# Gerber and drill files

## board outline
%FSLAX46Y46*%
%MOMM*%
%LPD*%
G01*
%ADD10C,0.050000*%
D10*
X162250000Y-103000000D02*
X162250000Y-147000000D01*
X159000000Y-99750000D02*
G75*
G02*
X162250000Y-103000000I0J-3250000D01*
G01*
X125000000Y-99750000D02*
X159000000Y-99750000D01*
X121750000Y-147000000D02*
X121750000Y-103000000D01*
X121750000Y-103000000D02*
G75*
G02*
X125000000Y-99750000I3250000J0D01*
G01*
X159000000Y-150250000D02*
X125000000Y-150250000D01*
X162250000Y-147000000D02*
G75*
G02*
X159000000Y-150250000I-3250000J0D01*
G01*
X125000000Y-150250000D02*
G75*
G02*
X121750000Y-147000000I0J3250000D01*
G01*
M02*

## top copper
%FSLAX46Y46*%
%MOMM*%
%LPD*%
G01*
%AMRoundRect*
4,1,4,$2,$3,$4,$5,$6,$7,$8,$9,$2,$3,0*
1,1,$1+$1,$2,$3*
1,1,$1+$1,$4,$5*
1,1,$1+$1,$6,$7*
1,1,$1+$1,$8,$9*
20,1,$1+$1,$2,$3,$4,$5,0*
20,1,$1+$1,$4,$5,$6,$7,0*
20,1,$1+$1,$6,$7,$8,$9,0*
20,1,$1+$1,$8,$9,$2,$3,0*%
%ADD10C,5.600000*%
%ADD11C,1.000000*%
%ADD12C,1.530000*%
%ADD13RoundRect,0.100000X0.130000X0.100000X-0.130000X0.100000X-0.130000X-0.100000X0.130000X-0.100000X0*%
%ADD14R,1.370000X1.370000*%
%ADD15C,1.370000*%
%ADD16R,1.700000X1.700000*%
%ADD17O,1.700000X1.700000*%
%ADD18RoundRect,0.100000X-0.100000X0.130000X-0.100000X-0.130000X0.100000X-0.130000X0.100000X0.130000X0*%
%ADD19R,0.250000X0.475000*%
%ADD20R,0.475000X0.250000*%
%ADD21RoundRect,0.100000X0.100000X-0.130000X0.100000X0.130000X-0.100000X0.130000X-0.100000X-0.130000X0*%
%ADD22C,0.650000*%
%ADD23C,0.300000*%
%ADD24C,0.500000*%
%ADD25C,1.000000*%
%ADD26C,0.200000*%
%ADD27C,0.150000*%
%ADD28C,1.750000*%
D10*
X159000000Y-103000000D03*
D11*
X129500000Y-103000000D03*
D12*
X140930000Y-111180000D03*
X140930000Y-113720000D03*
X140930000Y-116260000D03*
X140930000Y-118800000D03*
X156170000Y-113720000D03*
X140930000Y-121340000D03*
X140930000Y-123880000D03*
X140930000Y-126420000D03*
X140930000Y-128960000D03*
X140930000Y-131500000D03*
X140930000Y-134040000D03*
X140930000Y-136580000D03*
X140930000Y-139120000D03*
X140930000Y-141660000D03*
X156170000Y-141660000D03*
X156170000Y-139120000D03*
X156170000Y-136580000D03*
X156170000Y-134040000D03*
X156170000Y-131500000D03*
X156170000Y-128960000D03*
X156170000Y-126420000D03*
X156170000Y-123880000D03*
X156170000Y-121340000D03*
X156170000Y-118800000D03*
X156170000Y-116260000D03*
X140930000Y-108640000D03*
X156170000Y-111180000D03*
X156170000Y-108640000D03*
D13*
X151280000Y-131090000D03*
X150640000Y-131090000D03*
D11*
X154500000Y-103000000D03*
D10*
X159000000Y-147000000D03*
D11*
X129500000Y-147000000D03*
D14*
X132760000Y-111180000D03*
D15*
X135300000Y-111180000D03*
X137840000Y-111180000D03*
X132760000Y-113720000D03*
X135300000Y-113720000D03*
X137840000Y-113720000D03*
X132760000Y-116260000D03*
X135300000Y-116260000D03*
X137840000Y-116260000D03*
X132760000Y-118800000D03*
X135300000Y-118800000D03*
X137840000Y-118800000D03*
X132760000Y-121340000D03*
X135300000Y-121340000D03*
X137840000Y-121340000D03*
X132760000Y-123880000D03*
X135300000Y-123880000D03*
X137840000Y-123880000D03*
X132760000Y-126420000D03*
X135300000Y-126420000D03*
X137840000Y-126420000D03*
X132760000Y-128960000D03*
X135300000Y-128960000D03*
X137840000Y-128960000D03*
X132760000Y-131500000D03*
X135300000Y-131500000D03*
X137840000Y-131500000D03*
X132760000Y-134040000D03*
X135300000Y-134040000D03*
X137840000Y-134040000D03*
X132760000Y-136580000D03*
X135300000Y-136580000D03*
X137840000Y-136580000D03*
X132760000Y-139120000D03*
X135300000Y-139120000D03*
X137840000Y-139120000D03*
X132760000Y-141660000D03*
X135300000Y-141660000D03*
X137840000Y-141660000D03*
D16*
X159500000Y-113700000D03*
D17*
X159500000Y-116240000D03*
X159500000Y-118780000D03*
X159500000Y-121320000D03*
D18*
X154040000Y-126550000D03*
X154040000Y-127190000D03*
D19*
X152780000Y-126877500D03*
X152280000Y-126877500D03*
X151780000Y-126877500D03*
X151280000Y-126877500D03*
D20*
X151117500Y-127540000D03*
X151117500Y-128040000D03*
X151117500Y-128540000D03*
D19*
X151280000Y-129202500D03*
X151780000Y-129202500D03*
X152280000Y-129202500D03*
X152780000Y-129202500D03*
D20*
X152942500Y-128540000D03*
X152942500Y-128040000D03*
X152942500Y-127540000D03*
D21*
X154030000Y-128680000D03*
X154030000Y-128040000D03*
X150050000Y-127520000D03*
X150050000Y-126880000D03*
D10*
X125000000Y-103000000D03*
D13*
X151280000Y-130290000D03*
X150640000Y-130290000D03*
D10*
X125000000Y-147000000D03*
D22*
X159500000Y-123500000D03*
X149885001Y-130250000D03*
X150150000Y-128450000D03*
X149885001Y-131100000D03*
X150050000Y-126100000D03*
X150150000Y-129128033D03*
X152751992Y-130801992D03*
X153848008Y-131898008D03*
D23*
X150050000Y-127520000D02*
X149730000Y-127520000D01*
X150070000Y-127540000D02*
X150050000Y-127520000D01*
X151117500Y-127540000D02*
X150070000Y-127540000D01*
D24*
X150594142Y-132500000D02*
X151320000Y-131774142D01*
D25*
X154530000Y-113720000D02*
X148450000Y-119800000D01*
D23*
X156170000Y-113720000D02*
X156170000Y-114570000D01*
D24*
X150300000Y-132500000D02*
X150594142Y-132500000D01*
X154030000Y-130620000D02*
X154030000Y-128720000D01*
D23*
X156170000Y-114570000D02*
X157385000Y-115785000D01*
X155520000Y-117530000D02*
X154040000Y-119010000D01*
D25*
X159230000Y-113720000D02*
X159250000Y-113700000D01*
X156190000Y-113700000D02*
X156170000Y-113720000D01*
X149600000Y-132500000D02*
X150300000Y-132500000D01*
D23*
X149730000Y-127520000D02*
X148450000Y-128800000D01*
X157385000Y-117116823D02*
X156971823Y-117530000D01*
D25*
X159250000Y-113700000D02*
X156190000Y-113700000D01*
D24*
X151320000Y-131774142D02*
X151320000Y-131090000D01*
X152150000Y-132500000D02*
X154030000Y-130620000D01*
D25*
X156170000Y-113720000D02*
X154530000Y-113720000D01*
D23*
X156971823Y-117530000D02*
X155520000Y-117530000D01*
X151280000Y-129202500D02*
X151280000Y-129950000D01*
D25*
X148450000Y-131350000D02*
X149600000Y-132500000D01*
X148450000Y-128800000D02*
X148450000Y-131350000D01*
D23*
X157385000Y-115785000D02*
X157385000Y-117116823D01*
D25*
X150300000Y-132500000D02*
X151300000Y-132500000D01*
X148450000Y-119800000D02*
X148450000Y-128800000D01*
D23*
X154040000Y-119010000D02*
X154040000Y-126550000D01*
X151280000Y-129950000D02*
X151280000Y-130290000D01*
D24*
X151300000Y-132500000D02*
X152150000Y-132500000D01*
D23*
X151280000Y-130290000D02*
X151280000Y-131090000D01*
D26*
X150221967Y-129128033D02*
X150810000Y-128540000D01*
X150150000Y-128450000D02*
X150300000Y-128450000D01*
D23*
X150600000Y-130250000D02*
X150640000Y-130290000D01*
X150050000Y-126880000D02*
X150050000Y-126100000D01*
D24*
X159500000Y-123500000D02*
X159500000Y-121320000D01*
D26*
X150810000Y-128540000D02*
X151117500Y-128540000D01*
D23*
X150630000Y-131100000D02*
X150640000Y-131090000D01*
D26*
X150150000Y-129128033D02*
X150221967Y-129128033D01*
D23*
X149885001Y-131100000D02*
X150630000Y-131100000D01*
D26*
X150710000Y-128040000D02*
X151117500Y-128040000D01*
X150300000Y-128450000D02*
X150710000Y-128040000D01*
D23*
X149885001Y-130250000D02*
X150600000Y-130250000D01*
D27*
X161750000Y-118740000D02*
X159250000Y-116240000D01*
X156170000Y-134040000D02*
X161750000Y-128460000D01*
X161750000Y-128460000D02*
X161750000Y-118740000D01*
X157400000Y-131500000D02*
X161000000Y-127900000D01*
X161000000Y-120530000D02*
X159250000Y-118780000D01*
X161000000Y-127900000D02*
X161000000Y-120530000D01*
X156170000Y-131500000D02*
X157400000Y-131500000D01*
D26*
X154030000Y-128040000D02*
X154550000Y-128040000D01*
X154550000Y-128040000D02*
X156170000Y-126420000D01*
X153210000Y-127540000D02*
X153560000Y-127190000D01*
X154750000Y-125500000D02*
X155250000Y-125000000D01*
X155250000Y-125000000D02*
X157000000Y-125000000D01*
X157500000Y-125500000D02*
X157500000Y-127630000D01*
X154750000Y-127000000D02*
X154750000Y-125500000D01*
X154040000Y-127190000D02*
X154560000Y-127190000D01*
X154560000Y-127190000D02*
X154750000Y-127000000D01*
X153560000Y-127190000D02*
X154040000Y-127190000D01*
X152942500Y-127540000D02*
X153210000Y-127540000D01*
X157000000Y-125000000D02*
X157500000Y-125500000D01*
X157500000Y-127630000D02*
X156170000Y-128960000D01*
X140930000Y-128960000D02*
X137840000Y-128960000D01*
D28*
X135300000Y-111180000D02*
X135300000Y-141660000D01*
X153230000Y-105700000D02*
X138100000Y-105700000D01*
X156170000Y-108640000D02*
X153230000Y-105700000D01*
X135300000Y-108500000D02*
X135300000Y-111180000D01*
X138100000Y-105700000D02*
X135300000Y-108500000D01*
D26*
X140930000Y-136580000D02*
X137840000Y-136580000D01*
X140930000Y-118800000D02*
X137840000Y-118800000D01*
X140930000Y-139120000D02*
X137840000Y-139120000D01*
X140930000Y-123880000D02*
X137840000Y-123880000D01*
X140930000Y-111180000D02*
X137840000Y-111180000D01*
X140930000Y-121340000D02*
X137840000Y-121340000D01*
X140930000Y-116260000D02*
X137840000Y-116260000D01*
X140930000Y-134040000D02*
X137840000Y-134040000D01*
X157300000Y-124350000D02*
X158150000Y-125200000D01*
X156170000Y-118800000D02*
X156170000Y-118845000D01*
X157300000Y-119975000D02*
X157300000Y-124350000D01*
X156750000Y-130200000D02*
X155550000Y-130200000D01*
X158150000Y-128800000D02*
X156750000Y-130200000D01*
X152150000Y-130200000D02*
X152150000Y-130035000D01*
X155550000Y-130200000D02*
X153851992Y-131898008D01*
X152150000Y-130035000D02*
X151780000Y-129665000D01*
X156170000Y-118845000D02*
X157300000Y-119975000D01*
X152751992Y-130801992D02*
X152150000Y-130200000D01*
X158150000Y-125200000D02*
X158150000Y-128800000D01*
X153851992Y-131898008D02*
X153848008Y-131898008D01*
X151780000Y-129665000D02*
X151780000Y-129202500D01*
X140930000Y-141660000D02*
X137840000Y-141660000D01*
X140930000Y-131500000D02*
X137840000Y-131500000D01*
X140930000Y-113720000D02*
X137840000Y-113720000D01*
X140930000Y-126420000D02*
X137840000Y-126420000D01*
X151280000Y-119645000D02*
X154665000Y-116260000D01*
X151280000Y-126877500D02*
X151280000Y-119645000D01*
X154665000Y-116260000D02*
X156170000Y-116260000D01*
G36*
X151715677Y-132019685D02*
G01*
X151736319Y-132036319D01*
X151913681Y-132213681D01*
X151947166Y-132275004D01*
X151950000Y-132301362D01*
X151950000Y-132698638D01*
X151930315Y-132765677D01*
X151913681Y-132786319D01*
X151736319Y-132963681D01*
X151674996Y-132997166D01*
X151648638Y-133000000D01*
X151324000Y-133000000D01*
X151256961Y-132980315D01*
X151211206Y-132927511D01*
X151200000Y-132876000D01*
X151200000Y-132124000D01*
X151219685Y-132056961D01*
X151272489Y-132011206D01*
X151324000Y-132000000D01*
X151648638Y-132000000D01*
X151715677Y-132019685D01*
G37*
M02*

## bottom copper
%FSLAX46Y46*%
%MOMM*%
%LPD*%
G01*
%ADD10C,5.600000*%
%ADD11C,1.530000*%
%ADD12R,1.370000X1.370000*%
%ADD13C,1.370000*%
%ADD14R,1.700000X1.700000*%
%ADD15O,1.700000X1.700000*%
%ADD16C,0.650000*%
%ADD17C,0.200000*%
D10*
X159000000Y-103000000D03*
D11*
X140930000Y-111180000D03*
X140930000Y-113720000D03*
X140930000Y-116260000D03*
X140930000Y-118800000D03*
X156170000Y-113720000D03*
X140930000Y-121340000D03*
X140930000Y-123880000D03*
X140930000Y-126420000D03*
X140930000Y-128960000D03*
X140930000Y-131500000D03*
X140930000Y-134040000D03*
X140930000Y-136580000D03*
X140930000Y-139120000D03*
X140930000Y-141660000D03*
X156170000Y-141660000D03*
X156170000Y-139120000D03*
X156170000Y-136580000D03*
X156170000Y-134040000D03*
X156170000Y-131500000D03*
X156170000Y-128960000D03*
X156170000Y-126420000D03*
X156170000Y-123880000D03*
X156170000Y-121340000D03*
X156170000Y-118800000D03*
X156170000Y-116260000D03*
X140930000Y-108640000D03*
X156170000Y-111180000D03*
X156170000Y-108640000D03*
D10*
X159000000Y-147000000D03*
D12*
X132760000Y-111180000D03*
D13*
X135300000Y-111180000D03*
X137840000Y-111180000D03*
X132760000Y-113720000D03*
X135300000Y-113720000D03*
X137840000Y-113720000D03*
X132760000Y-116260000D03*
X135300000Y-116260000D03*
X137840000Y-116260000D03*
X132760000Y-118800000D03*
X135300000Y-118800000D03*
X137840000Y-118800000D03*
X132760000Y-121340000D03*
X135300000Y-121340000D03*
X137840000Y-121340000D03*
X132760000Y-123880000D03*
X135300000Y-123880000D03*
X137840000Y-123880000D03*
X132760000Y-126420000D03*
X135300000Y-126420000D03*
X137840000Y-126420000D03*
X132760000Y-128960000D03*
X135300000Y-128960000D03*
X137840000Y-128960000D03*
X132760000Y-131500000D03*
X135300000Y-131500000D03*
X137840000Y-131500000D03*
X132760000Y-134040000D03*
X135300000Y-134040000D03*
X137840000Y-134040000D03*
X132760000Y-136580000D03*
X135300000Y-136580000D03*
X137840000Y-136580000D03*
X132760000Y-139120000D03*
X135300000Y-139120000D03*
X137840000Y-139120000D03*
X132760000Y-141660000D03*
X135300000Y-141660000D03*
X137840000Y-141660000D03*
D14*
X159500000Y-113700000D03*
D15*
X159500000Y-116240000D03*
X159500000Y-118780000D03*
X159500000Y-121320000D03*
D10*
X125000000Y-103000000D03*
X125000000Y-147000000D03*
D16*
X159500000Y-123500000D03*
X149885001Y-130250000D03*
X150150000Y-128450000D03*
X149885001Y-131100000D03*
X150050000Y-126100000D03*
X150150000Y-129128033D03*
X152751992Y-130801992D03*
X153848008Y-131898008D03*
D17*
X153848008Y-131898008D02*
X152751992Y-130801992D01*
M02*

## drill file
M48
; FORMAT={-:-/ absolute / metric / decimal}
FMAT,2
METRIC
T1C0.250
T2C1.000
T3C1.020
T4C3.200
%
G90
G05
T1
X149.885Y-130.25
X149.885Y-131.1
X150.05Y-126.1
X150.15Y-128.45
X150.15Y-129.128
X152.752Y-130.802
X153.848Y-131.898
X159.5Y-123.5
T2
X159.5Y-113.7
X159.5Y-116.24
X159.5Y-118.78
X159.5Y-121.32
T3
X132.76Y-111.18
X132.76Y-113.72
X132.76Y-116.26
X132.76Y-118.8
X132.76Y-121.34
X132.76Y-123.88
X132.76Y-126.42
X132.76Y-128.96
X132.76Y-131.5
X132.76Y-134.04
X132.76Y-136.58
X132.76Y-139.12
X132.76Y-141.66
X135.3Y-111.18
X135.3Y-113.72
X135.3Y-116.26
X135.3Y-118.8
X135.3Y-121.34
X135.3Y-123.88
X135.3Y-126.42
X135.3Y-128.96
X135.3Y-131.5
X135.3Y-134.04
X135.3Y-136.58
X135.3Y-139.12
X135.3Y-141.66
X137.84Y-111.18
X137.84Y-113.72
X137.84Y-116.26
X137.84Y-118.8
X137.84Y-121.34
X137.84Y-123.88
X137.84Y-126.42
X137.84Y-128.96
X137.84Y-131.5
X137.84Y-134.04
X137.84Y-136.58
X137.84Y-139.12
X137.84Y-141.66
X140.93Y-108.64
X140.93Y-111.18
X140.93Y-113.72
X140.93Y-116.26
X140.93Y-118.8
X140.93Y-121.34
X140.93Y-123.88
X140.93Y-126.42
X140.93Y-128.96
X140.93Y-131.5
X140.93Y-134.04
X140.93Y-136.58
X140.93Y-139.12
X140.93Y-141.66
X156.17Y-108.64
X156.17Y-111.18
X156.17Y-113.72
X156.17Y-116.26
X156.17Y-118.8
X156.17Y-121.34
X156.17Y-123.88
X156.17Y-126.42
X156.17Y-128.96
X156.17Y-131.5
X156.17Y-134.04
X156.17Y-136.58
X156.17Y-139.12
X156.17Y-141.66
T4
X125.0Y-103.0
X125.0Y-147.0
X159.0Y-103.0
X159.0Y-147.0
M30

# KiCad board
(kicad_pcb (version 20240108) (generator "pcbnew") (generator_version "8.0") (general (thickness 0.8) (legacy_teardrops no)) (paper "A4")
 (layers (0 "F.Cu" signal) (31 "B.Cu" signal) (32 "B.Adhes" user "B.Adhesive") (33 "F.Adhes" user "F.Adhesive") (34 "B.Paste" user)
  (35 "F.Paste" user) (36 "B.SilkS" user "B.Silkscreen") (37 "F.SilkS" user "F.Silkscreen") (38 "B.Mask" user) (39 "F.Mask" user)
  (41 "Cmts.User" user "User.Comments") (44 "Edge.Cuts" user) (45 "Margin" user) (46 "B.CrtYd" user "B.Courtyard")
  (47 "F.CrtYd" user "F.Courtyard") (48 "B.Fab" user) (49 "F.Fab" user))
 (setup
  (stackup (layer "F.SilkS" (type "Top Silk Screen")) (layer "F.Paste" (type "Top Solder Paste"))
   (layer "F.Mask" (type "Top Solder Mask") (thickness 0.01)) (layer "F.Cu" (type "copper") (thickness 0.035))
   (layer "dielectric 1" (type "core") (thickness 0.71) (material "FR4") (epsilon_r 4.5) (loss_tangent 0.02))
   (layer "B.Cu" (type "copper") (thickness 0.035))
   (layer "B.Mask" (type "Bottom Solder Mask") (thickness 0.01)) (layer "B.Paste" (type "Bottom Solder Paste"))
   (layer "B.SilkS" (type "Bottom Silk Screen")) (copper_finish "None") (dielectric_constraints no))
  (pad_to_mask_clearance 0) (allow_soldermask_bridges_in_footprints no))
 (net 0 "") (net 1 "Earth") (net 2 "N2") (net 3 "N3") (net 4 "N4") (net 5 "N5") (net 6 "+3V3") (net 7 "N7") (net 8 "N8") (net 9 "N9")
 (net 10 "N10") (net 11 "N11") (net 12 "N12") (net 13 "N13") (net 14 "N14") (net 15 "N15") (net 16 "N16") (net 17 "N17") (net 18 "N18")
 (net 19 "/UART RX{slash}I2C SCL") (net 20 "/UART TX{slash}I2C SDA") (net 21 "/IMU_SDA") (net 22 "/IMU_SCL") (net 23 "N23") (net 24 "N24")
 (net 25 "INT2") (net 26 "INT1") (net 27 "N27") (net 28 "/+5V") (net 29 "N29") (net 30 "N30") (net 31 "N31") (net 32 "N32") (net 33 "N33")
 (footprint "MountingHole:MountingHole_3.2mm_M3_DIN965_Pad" (layer "F.Cu") (at 159 103)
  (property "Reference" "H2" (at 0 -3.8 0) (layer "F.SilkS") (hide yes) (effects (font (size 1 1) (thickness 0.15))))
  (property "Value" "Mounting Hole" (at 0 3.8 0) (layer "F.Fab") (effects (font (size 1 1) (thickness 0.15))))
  (pad "1" thru_hole circle (at 0 0) (size 5.6 5.6) (drill 3.2) (layers "*.Cu" "*.Mask") (remove_unused_layers no) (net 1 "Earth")))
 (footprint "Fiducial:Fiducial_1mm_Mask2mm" (layer "F.Cu") (at 129.5 103)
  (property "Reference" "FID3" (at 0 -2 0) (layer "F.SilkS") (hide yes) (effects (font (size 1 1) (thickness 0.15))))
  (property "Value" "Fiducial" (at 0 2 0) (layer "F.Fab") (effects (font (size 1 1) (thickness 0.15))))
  (pad "" smd circle (at 0 0) (size 1 1) (layers "F.Cu" "F.Mask") (solder_mask_margin 0.5) (clearance 0.5)))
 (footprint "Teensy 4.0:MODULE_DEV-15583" (layer "F.Cu") (at 148.55 125.15)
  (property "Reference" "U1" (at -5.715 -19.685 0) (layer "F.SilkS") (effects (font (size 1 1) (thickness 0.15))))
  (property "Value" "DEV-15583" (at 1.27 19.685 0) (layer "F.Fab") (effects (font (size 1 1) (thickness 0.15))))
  (pad "0" thru_hole circle (at -7.62 -13.97) (size 1.53 1.53) (drill 1.02) (layers "*.Cu" "*.Mask") (remove_unused_layers no) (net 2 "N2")
   (solder_mask_margin 0.102))
  (pad "1" thru_hole circle (at -7.62 -11.43) (size 1.53 1.53) (drill 1.02) (layers "*.Cu" "*.Mask") (remove_unused_layers no) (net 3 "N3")
   (solder_mask_margin 0.102))
  (pad "2" thru_hole circle (at -7.62 -8.89) (size 1.53 1.53) (drill 1.02) (layers "*.Cu" "*.Mask") (remove_unused_layers no) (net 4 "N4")
   (solder_mask_margin 0.102))
  (pad "3" thru_hole circle (at -7.62 -6.35) (size 1.53 1.53) (drill 1.02) (layers "*.Cu" "*.Mask") (remove_unused_layers no) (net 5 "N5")
   (solder_mask_margin 0.102))
  (pad "3v3" thru_hole circle (at 7.62 -11.43) (size 1.53 1.53) (drill 1.02) (layers "*.Cu" "*.Mask") (remove_unused_layers no)
   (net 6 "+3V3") (solder_mask_margin 0.102))
  (pad "4" thru_hole circle (at -7.62 -3.81) (size 1.53 1.53) (drill 1.02) (layers "*.Cu" "*.Mask") (remove_unused_layers no) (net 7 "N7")
   (solder_mask_margin 0.102))
  (pad "5" thru_hole circle (at -7.62 -1.27) (size 1.53 1.53) (drill 1.02) (layers "*.Cu" "*.Mask") (remove_unused_layers no) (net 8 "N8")
   (solder_mask_margin 0.102))
  (pad "6" thru_hole circle (at -7.62 1.27) (size 1.53 1.53) (drill 1.02) (layers "*.Cu" "*.Mask") (remove_unused_layers no) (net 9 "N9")
   (solder_mask_margin 0.102))
  (pad "7" thru_hole circle (at -7.62 3.81) (size 1.53 1.53) (drill 1.02) (layers "*.Cu" "*.Mask") (remove_unused_layers no) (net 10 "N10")
   (solder_mask_margin 0.102))
  (pad "8" thru_hole circle (at -7.62 6.35) (size 1.53 1.53) (drill 1.02) (layers "*.Cu" "*.Mask") (remove_unused_layers no) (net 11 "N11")
   (solder_mask_margin 0.102))
  (pad "9" thru_hole circle (at -7.62 8.89) (size 1.53 1.53) (drill 1.02) (layers "*.Cu" "*.Mask") (remove_unused_layers no) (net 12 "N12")
   (solder_mask_margin 0.102))
  (pad "10" thru_hole circle (at -7.62 11.43) (size 1.53 1.53) (drill 1.02) (layers "*.Cu" "*.Mask") (remove_unused_layers no)
   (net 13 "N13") (solder_mask_margin 0.102))
  (pad "11" thru_hole circle (at -7.62 13.97) (size 1.53 1.53) (drill 1.02) (layers "*.Cu" "*.Mask") (remove_unused_layers no)
   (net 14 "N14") (solder_mask_margin 0.102))
  (pad "12" thru_hole circle (at -7.62 16.51) (size 1.53 1.53) (drill 1.02) (layers "*.Cu" "*.Mask") (remove_unused_layers no)
   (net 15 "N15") (solder_mask_margin 0.102))
  (pad "13" thru_hole circle (at 7.62 16.51) (size 1.53 1.53) (drill 1.02) (layers "*.Cu" "*.Mask") (remove_unused_layers no) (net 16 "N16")
   (solder_mask_margin 0.102))
  (pad "14" thru_hole circle (at 7.62 13.97) (size 1.53 1.53) (drill 1.02) (layers "*.Cu" "*.Mask") (remove_unused_layers no) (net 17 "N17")
   (solder_mask_margin 0.102))
  (pad "15" thru_hole circle (at 7.62 11.43) (size 1.53 1.53) (drill 1.02) (layers "*.Cu" "*.Mask") (remove_unused_layers no) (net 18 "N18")
   (solder_mask_margin 0.102))
  (pad "16" thru_hole circle (at 7.62 8.89) (size 1.53 1.53) (drill 1.02) (layers "*.Cu" "*.Mask") (remove_unused_layers no)
   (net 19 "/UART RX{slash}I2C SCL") (solder_mask_margin 0.102))
  (pad "17" thru_hole circle (at 7.62 6.35) (size 1.53 1.53) (drill 1.02) (layers "*.Cu" "*.Mask") (remove_unused_layers no)
   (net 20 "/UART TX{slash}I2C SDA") (solder_mask_margin 0.102))
  (pad "18" thru_hole circle (at 7.62 3.81) (size 1.53 1.53) (drill 1.02) (layers "*.Cu" "*.Mask") (remove_unused_layers no)
   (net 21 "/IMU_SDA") (solder_mask_margin 0.102))
  (pad "19" thru_hole circle (at 7.62 1.27) (size 1.53 1.53) (drill 1.02) (layers "*.Cu" "*.Mask") (remove_unused_layers no)
   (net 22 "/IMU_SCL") (solder_mask_margin 0.102))
  (pad "20" thru_hole circle (at 7.62 -1.27) (size 1.53 1.53) (drill 1.02) (layers "*.Cu" "*.Mask") (remove_unused_layers no) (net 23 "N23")
   (solder_mask_margin 0.102))
  (pad "21" thru_hole circle (at 7.62 -3.81) (size 1.53 1.53) (drill 1.02) (layers "*.Cu" "*.Mask") (remove_unused_layers no) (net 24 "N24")
   (solder_mask_margin 0.102))
  (pad "22" thru_hole circle (at 7.62 -6.35) (size 1.53 1.53) (drill 1.02) (layers "*.Cu" "*.Mask") (remove_unused_layers no)
   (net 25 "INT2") (solder_mask_margin 0.102))
  (pad "23" thru_hole circle (at 7.62 -8.89) (size 1.53 1.53) (drill 1.02) (layers "*.Cu" "*.Mask") (remove_unused_layers no)
   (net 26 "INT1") (solder_mask_margin 0.102))
  (pad "G1" thru_hole circle (at -7.62 -16.51) (size 1.53 1.53) (drill 1.02) (layers "*.Cu" "*.Mask") (remove_unused_layers no)
   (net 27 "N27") (solder_mask_margin 0.102))
  (pad "G3" thru_hole circle (at 7.62 -13.97) (size 1.53 1.53) (drill 1.02) (layers "*.Cu" "*.Mask") (remove_unused_layers no)
   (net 1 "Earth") (solder_mask_margin 0.102))
  (pad "VIN" thru_hole circle (at 7.62 -16.51) (size 1.53 1.53) (drill 1.02) (layers "*.Cu" "*.Mask") (remove_unused_layers no)
   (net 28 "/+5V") (solder_mask_margin 0.102)))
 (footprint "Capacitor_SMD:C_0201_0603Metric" (layer "F.Cu") (at 150.96 131.09 180)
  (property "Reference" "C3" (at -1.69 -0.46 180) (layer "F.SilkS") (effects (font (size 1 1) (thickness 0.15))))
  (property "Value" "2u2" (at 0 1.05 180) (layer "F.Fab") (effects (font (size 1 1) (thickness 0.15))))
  (pad "" smd roundrect (at -0.345 0 180) (size 0.318 0.36) (layers "F.Paste") (roundrect_rratio 0.25))
  (pad "" smd roundrect (at 0.345 0 180) (size 0.318 0.36) (layers "F.Paste") (roundrect_rratio 0.25))
  (pad "1" smd roundrect (at -0.32 0 180) (size 0.46 0.4) (layers "F.Cu" "F.Mask") (roundrect_rratio 0.25) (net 6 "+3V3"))
  (pad "2" smd roundrect (at 0.32 0 180) (size 0.46 0.4) (layers "F.Cu" "F.Mask") (roundrect_rratio 0.25) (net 1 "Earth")))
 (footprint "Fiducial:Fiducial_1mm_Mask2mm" (layer "F.Cu") (at 154.5 103)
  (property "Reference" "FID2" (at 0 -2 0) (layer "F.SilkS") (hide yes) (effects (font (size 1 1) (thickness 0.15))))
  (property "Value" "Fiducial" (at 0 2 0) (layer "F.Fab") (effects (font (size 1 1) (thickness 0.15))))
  (pad "" smd circle (at 0 0) (size 1 1) (layers "F.Cu" "F.Mask") (solder_mask_margin 0.5) (clearance 0.5)))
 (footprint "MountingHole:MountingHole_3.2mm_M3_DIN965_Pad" (layer "F.Cu") (at 159 147)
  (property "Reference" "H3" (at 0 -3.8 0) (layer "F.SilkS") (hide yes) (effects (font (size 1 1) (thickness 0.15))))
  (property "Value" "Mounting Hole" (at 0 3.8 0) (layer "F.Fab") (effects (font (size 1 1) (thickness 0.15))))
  (pad "1" thru_hole circle (at 0 0) (size 5.6 5.6) (drill 3.2) (layers "*.Cu" "*.Mask") (remove_unused_layers no) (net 1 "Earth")))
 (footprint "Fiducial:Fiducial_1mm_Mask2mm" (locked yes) (layer "F.Cu") (at 129.5 147)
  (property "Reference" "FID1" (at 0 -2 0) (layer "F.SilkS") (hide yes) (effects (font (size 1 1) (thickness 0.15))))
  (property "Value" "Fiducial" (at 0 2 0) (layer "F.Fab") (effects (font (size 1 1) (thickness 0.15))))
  (pad "" smd circle (at 0 0) (size 1 1) (layers "F.Cu" "F.Mask") (solder_mask_margin 0.5) (clearance 0.5)))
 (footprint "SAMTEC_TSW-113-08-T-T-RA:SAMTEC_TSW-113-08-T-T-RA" (layer "F.Cu") (at 129.99 126.42 -90)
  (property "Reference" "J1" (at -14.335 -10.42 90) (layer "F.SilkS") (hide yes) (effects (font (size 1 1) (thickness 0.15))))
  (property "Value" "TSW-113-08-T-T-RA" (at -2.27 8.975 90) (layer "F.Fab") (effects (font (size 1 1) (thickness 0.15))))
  (pad "01" thru_hole rect (at -15.24 -2.77 270) (size 1.37 1.37) (drill 1.02) (layers "*.Cu" "*.Mask") (remove_unused_layers no)
   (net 27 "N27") (solder_mask_margin 0.102))
  (pad "02" thru_hole circle (at -15.24 -5.31 270) (size 1.37 1.37) (drill 1.02) (layers "*.Cu" "*.Mask") (remove_unused_layers no)
   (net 28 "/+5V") (solder_mask_margin 0.102))
  (pad "03" thru_hole circle (at -15.24 -7.85 270) (size 1.37 1.37) (drill 1.02) (layers "*.Cu" "*.Mask") (remove_unused_layers no)
   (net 2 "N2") (solder_mask_margin 0.102))
  (pad "04" thru_hole circle (at -12.7 -2.77 270) (size 1.37 1.37) (drill 1.02) (layers "*.Cu" "*.Mask") (remove_unused_layers no)
   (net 27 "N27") (solder_mask_margin 0.102))
  (pad "05" thru_hole circle (at -12.7 -5.31 270) (size 1.37 1.37) (drill 1.02) (layers "*.Cu" "*.Mask") (remove_unused_layers no)
   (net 28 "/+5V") (solder_mask_margin 0.102))
  (pad "06" thru_hole circle (at -12.7 -7.85 270) (size 1.37 1.37) (drill 1.02) (layers "*.Cu" "*.Mask") (remove_unused_layers no)
   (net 3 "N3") (solder_mask_margin 0.102))
  (pad "07" thru_hole circle (at -10.16 -2.77 270) (size 1.37 1.37) (drill 1.02) (layers "*.Cu" "*.Mask") (remove_unused_layers no)
   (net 27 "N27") (solder_mask_margin 0.102))
  (pad "08" thru_hole circle (at -10.16 -5.31 270) (size 1.37 1.37) (drill 1.02) (layers "*.Cu" "*.Mask") (remove_unused_layers no)
   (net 28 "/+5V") (solder_mask_margin 0.102))
  (pad "09" thru_hole circle (at -10.16 -7.85 270) (size 1.37 1.37) (drill 1.02) (layers "*.Cu" "*.Mask") (remove_unused_layers no)
   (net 4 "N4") (solder_mask_margin 0.102))
  (pad "10" thru_hole circle (at -7.62 -2.77 270) (size 1.37 1.37) (drill 1.02) (layers "*.Cu" "*.Mask") (remove_unused_layers no)
   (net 27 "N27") (solder_mask_margin 0.102))
  (pad "11" thru_hole circle (at -7.62 -5.31 270) (size 1.37 1.37) (drill 1.02) (layers "*.Cu" "*.Mask") (remove_unused_layers no)
   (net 28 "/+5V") (solder_mask_margin 0.102))
  (pad "12" thru_hole circle (at -7.62 -7.85 270) (size 1.37 1.37) (drill 1.02) (layers "*.Cu" "*.Mask") (remove_unused_layers no)
   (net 5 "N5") (solder_mask_margin 0.102))
  (pad "13" thru_hole circle (at -5.08 -2.77 270) (size 1.37 1.37) (drill 1.02) (layers "*.Cu" "*.Mask") (remove_unused_layers no)
   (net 27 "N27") (solder_mask_margin 0.102))
  (pad "14" thru_hole circle (at -5.08 -5.31 270) (size 1.37 1.37) (drill 1.02) (layers "*.Cu" "*.Mask") (remove_unused_layers no)
   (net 28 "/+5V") (solder_mask_margin 0.102))
  (pad "15" thru_hole circle (at -5.08 -7.85 270) (size 1.37 1.37) (drill 1.02) (layers "*.Cu" "*.Mask") (remove_unused_layers no)
   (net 7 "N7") (solder_mask_margin 0.102))
  (pad "16" thru_hole circle (at -2.54 -2.77 270) (size 1.37 1.37) (drill 1.02) (layers "*.Cu" "*.Mask") (remove_unused_layers no)
   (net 27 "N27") (solder_mask_margin 0.102))
  (pad "17" thru_hole circle (at -2.54 -5.31 270) (size 1.37 1.37) (drill 1.02) (layers "*.Cu" "*.Mask") (remove_unused_layers no)
   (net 28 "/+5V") (solder_mask_margin 0.102))
  (pad "18" thru_hole circle (at -2.54 -7.85 270) (size 1.37 1.37) (drill 1.02) (layers "*.Cu" "*.Mask") (remove_unused_layers no)
   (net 8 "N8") (solder_mask_margin 0.102))
  (pad "19" thru_hole circle (at 0 -2.77 270) (size 1.37 1.37) (drill 1.02) (layers "*.Cu" "*.Mask") (remove_unused_layers no)
   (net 27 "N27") (solder_mask_margin 0.102))
  (pad "20" thru_hole circle (at 0 -5.31 270) (size 1.37 1.37) (drill 1.02) (layers "*.Cu" "*.Mask") (remove_unused_layers no)
   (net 28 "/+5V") (solder_mask_margin 0.102))
  (pad "21" thru_hole circle (at 0 -7.85 270) (size 1.37 1.37) (drill 1.02) (layers "*.Cu" "*.Mask") (remove_unused_layers no) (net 9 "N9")
   (solder_mask_margin 0.102))
  (pad "22" thru_hole circle (at 2.54 -2.77 270) (size 1.37 1.37) (drill 1.02) (layers "*.Cu" "*.Mask") (remove_unused_layers no)
   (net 27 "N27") (solder_mask_margin 0.102))
  (pad "23" thru_hole circle (at 2.54 -5.31 270) (size 1.37 1.37) (drill 1.02) (layers "*.Cu" "*.Mask") (remove_unused_layers no)
   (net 28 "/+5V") (solder_mask_margin 0.102))
  (pad "24" thru_hole circle (at 2.54 -7.85 270) (size 1.37 1.37) (drill 1.02) (layers "*.Cu" "*.Mask") (remove_unused_layers no)
   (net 10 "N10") (solder_mask_margin 0.102))
  (pad "25" thru_hole circle (at 5.08 -2.77 270) (size 1.37 1.37) (drill 1.02) (layers "*.Cu" "*.Mask") (remove_unused_layers no)
   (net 27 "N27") (solder_mask_margin 0.102))
  (pad "26" thru_hole circle (at 5.08 -5.31 270) (size 1.37 1.37) (drill 1.02) (layers "*.Cu" "*.Mask") (remove_unused_layers no)
   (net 28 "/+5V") (solder_mask_margin 0.102))
  (pad "27" thru_hole circle (at 5.08 -7.85 270) (size 1.37 1.37) (drill 1.02) (layers "*.Cu" "*.Mask") (remove_unused_layers no)
   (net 11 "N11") (solder_mask_margin 0.102))
  (pad "28" thru_hole circle (at 7.62 -2.77 270) (size 1.37 1.37) (drill 1.02) (layers "*.Cu" "*.Mask") (remove_unused_layers no)
   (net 27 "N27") (solder_mask_margin 0.102))
  (pad "29" thru_hole circle (at 7.62 -5.31 270) (size 1.37 1.37) (drill 1.02) (layers "*.Cu" "*.Mask") (remove_unused_layers no)
   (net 28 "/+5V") (solder_mask_margin 0.102))
  (pad "30" thru_hole circle (at 7.62 -7.85 270) (size 1.37 1.37) (drill 1.02) (layers "*.Cu" "*.Mask") (remove_unused_layers no)
   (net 12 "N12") (solder_mask_margin 0.102))
  (pad "31" thru_hole circle (at 10.16 -2.77 270) (size 1.37 1.37) (drill 1.02) (layers "*.Cu" "*.Mask") (remove_unused_layers no)
   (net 27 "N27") (solder_mask_margin 0.102))
  (pad "32" thru_hole circle (at 10.16 -5.31 270) (size 1.37 1.37) (drill 1.02) (layers "*.Cu" "*.Mask") (remove_unused_layers no)
   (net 28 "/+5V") (solder_mask_margin 0.102))
  (pad "33" thru_hole circle (at 10.16 -7.85 270) (size 1.37 1.37) (drill 1.02) (layers "*.Cu" "*.Mask") (remove_unused_layers no)
   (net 13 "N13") (solder_mask_margin 0.102))
  (pad "34" thru_hole circle (at 12.7 -2.77 270) (size 1.37 1.37) (drill 1.02) (layers "*.Cu" "*.Mask") (remove_unused_layers no)
   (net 27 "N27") (solder_mask_margin 0.102))
  (pad "35" thru_hole circle (at 12.7 -5.31 270) (size 1.37 1.37) (drill 1.02) (layers "*.Cu" "*.Mask") (remove_unused_layers no)
   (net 28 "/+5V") (solder_mask_margin 0.102))
  (pad "36" thru_hole circle (at 12.7 -7.85 270) (size 1.37 1.37) (drill 1.02) (layers "*.Cu" "*.Mask") (remove_unused_layers no)
   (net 14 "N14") (solder_mask_margin 0.102))
  (pad "37" thru_hole circle (at 15.24 -2.77 270) (size 1.37 1.37) (drill 1.02) (layers "*.Cu" "*.Mask") (remove_unused_layers no)
   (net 27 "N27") (solder_mask_margin 0.102))
  (pad "38" thru_hole circle (at 15.24 -5.31 270) (size 1.37 1.37) (drill 1.02) (layers "*.Cu" "*.Mask") (remove_unused_layers no)
   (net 28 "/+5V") (solder_mask_margin 0.102))
  (pad "39" thru_hole circle (at 15.24 -7.85 270) (size 1.37 1.37) (drill 1.02) (layers "*.Cu" "*.Mask") (remove_unused_layers no)
   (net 15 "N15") (solder_mask_margin 0.102)))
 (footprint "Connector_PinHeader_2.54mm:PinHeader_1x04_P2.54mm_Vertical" (layer "F.Cu") (at 159.5 113.7)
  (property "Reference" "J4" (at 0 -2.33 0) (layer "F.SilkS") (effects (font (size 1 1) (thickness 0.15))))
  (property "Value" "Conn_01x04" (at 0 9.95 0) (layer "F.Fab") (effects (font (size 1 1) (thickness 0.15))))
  (pad "1" thru_hole rect (at 0 0) (size 1.7 1.7) (drill 1) (layers "*.Cu" "*.Mask") (remove_unused_layers no) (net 6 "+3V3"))
  (pad "2" thru_hole oval (at 0 2.54) (size 1.7 1.7) (drill 1) (layers "*.Cu" "*.Mask") (remove_unused_layers no)
   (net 19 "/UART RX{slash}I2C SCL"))
  (pad "3" thru_hole oval (at 0 5.08) (size 1.7 1.7) (drill 1) (layers "*.Cu" "*.Mask") (remove_unused_layers no)
   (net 20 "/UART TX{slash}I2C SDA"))
  (pad "4" thru_hole oval (at 0 7.62) (size 1.7 1.7) (drill 1) (layers "*.Cu" "*.Mask") (remove_unused_layers no) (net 1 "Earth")))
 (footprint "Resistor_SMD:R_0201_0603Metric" (layer "F.Cu") (at 154.04 126.87 -90)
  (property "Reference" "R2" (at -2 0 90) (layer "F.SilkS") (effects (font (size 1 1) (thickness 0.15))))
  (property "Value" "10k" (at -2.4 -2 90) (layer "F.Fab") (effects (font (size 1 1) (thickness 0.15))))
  (pad "" smd roundrect (at -0.345 0 270) (size 0.318 0.36) (layers "F.Paste") (roundrect_rratio 0.25))
  (pad "" smd roundrect (at 0.345 0 270) (size 0.318 0.36) (layers "F.Paste") (roundrect_rratio 0.25))
  (pad "1" smd roundrect (at -0.32 0 270) (size 0.46 0.4) (layers "F.Cu" "F.Mask") (roundrect_rratio 0.25) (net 6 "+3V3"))
  (pad "2" smd roundrect (at 0.32 0 270) (size 0.46 0.4) (layers "F.Cu" "F.Mask") (roundrect_rratio 0.25) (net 21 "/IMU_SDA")))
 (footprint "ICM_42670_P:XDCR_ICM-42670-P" (layer "F.Cu") (at 152.03 128.04 -90)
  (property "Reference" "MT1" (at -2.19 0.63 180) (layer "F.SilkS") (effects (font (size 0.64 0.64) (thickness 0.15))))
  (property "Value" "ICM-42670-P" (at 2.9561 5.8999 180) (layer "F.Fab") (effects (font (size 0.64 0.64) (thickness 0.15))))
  (pad "1" smd rect (at -1.1625 -0.75 270) (size 0.475 0.25) (layers "F.Cu") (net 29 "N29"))
  (pad "2" smd rect (at -1.1625 -0.25 270) (size 0.475 0.25) (layers "F.Cu") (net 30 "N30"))
  (pad "3" smd rect (at -1.1625 0.25 270) (size 0.475 0.25) (layers "F.Cu") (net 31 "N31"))
  (pad "4" smd rect (at -1.1625 0.75 270) (size 0.475 0.25) (layers "F.Cu") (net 26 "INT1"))
  (pad "5" smd rect (at -0.5 0.9125 270) (size 0.25 0.475) (layers "F.Cu") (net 6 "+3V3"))
  (pad "6" smd rect (at 0 0.9125 270) (size 0.25 0.475) (layers "F.Cu") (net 1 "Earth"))
  (pad "7" smd rect (at 0.5 0.9125 270) (size 0.25 0.475) (layers "F.Cu") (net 1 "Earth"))
  (pad "8" smd rect (at 1.1625 0.75 270) (size 0.475 0.25) (layers "F.Cu") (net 6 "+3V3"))
  (pad "9" smd rect (at 1.1625 0.25 270) (size 0.475 0.25) (layers "F.Cu") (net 25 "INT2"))
  (pad "10" smd rect (at 1.1625 -0.25 270) (size 0.475 0.25) (layers "F.Cu") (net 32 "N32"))
  (pad "11" smd rect (at 1.1625 -0.75 270) (size 0.475 0.25) (layers "F.Cu") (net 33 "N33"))
  (pad "12" smd rect (at 0.5 -0.9125 270) (size 0.25 0.475) (layers "F.Cu") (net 6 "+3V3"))
  (pad "13" smd rect (at 0 -0.9125 270) (size 0.25 0.475) (layers "F.Cu") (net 22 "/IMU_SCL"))
  (pad "14" smd rect (at -0.5 -0.9125 270) (size 0.25 0.475) (layers "F.Cu") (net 21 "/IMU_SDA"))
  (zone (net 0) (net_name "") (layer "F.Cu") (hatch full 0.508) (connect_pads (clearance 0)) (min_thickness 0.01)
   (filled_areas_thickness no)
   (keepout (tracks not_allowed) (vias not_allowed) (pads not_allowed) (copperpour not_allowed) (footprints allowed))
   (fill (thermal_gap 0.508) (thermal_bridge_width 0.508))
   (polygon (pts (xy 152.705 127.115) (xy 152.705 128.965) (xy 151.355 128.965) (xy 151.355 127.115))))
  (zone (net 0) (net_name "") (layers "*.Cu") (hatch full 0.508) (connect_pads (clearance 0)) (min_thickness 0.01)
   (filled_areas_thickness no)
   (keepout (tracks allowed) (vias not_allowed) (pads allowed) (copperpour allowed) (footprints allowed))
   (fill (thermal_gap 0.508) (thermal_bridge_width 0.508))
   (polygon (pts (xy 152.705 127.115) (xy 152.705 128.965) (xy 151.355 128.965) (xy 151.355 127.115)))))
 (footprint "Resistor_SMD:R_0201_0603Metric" (layer "F.Cu") (at 154.03 128.36 90)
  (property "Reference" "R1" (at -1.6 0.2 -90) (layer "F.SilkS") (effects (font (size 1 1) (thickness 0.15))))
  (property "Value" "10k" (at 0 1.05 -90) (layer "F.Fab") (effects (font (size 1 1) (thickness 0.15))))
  (pad "" smd roundrect (at -0.345 0 90) (size 0.318 0.36) (layers "F.Paste") (roundrect_rratio 0.25))
  (pad "" smd roundrect (at 0.345 0 90) (size 0.318 0.36) (layers "F.Paste") (roundrect_rratio 0.25))
  (pad "1" smd roundrect (at -0.32 0 90) (size 0.46 0.4) (layers "F.Cu" "F.Mask") (roundrect_rratio 0.25) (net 6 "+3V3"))
  (pad "2" smd roundrect (at 0.32 0 90) (size 0.46 0.4) (layers "F.Cu" "F.Mask") (roundrect_rratio 0.25) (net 22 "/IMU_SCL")))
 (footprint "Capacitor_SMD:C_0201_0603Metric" (layer "F.Cu") (at 150.05 127.2 90)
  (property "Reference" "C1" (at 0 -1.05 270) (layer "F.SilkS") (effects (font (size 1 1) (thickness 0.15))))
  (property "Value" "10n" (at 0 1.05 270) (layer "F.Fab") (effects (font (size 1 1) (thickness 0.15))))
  (pad "" smd roundrect (at -0.345 0 90) (size 0.318 0.36) (layers "F.Paste") (roundrect_rratio 0.25))
  (pad "" smd roundrect (at 0.345 0 90) (size 0.318 0.36) (layers "F.Paste") (roundrect_rratio 0.25))
  (pad "1" smd roundrect (at -0.32 0 90) (size 0.46 0.4) (layers "F.Cu" "F.Mask") (roundrect_rratio 0.25) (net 6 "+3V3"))
  (pad "2" smd roundrect (at 0.32 0 90) (size 0.46 0.4) (layers "F.Cu" "F.Mask") (roundrect_rratio 0.25) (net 1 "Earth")))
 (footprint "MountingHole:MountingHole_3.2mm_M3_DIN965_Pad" (layer "F.Cu") (at 125 103)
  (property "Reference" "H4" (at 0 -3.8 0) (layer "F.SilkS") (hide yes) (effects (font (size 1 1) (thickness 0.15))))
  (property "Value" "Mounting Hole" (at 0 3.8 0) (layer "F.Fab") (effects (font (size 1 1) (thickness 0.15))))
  (pad "1" thru_hole circle (at 0 0) (size 5.6 5.6) (drill 3.2) (layers "*.Cu" "*.Mask") (remove_unused_layers no) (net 1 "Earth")))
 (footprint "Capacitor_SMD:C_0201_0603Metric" (layer "F.Cu") (at 150.96 130.29 180)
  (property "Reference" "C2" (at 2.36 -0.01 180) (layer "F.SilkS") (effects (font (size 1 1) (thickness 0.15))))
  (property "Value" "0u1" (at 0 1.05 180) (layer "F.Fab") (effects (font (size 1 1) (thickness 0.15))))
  (pad "" smd roundrect (at -0.345 0 180) (size 0.318 0.36) (layers "F.Paste") (roundrect_rratio 0.25))
  (pad "" smd roundrect (at 0.345 0 180) (size 0.318 0.36) (layers "F.Paste") (roundrect_rratio 0.25))
  (pad "1" smd roundrect (at -0.32 0 180) (size 0.46 0.4) (layers "F.Cu" "F.Mask") (roundrect_rratio 0.25) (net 6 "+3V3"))
  (pad "2" smd roundrect (at 0.32 0 180) (size 0.46 0.4) (layers "F.Cu" "F.Mask") (roundrect_rratio 0.25) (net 1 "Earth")))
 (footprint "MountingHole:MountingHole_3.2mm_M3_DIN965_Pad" (layer "F.Cu") (at 125 147)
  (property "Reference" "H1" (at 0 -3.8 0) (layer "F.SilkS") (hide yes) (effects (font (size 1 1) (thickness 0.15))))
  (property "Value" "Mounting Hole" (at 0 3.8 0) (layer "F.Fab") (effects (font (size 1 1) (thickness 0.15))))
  (pad "1" thru_hole circle (at 0 0) (size 5.6 5.6) (drill 3.2) (layers "*.Cu" "*.Mask") (remove_unused_layers no) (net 1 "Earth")))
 (gr_line (start 162.25 103) (end 162.25 147) (stroke (width 0.05) (type default)) (layer "Edge.Cuts"))
 (gr_arc (start 159 99.75) (mid 161.298097 100.701903) (end 162.25 103) (stroke (width 0.05) (type default)) (layer "Edge.Cuts"))
 (gr_line (start 125 99.75) (end 159 99.75) (stroke (width 0.05) (type default)) (layer "Edge.Cuts"))
 (gr_line (start 121.75 147) (end 121.75 103) (stroke (width 0.05) (type default)) (layer "Edge.Cuts"))
 (gr_arc (start 121.75 103) (mid 122.701903 100.701903) (end 125 99.75) (stroke (width 0.05) (type default)) (layer "Edge.Cuts"))
 (gr_line (start 159 150.25) (end 125 150.25) (stroke (width 0.05) (type default)) (layer "Edge.Cuts"))
 (gr_arc (start 162.25 147) (mid 161.298097 149.298097) (end 159 150.25) (stroke (width 0.05) (type default)) (layer "Edge.Cuts"))
 (gr_arc (start 125 150.25) (mid 122.701903 149.298097) (end 121.75 147) (stroke (width 0.05) (type default)) (layer "Edge.Cuts"))
 (segment (start 150.05 127.52) (end 149.73 127.52) (width 0.3) (layer "F.Cu") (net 6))
 (segment (start 150.07 127.54) (end 150.05 127.52) (width 0.3) (layer "F.Cu") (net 6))
 (segment (start 151.1175 127.54) (end 150.07 127.54) (width 0.3) (layer "F.Cu") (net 6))
 (segment (start 150.594142 132.5) (end 151.32 131.774142) (width 0.5) (layer "F.Cu") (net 6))
 (segment (start 154.53 113.72) (end 148.45 119.8) (width 1) (layer "F.Cu") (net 6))
 (segment (start 156.17 113.72) (end 156.17 114.57) (width 0.3) (layer "F.Cu") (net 6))
 (segment (start 150.3 132.5) (end 150.594142 132.5) (width 0.5) (layer "F.Cu") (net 6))
 (segment (start 154.03 130.62) (end 154.03 128.72) (width 0.5) (layer "F.Cu") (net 6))
 (segment (start 156.17 114.57) (end 157.385 115.785) (width 0.3) (layer "F.Cu") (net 6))
 (segment (start 155.52 117.53) (end 154.04 119.01) (width 0.3) (layer "F.Cu") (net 6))
 (segment (start 159.23 113.72) (end 159.25 113.7) (width 1) (layer "F.Cu") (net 6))
 (segment (start 156.19 113.7) (end 156.17 113.72) (width 1) (layer "F.Cu") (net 6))
 (segment (start 149.6 132.5) (end 150.3 132.5) (width 1) (layer "F.Cu") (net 6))
 (segment (start 149.73 127.52) (end 148.45 128.8) (width 0.3) (layer "F.Cu") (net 6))
 (segment (start 157.385 117.116823) (end 156.971823 117.53) (width 0.3) (layer "F.Cu") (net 6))
 (segment (start 159.25 113.7) (end 156.19 113.7) (width 1) (layer "F.Cu") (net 6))
 (segment (start 151.32 131.774142) (end 151.32 131.09) (width 0.5) (layer "F.Cu") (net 6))
 (segment (start 152.15 132.5) (end 154.03 130.62) (width 0.5) (layer "F.Cu") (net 6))
 (segment (start 156.17 113.72) (end 154.53 113.72) (width 1) (layer "F.Cu") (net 6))
 (segment (start 156.971823 117.53) (end 155.52 117.53) (width 0.3) (layer "F.Cu") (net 6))
 (segment (start 151.28 129.2025) (end 151.28 129.95) (width 0.3) (layer "F.Cu") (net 6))
 (segment (start 148.45 131.35) (end 149.6 132.5) (width 1) (layer "F.Cu") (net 6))
 (segment (start 148.45 128.8) (end 148.45 131.35) (width 1) (layer "F.Cu") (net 6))
 (segment (start 157.385 115.785) (end 157.385 117.116823) (width 0.3) (layer "F.Cu") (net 6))
 (segment (start 150.3 132.5) (end 151.3 132.5) (width 1) (layer "F.Cu") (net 6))
 (segment (start 148.45 119.8) (end 148.45 128.8) (width 1) (layer "F.Cu") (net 6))
 (segment (start 154.04 119.01) (end 154.04 126.55) (width 0.3) (layer "F.Cu") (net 6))
 (segment (start 151.28 129.95) (end 151.28 130.29) (width 0.3) (layer "F.Cu") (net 6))
 (segment (start 151.3 132.5) (end 152.15 132.5) (width 0.5) (layer "F.Cu") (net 6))
 (segment (start 151.28 130.29) (end 151.28 131.09) (width 0.3) (layer "F.Cu") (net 6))
 (segment (start 150.221967 129.128033) (end 150.81 128.54) (width 0.2) (layer "F.Cu") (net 1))
 (segment (start 150.15 128.45) (end 150.3 128.45) (width 0.2) (layer "F.Cu") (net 1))
 (segment (start 150.6 130.25) (end 150.64 130.29) (width 0.3) (layer "F.Cu") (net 1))
 (segment (start 150.05 126.88) (end 150.05 126.1) (width 0.3) (layer "F.Cu") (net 1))
 (segment (start 159.5 123.5) (end 159.5 121.32) (width 0.5) (layer "F.Cu") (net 1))
 (segment (start 150.81 128.54) (end 151.1175 128.54) (width 0.2) (layer "F.Cu") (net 1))
 (segment (start 150.63 131.1) (end 150.64 131.09) (width 0.3) (layer "F.Cu") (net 1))
 (segment (start 150.15 129.128033) (end 150.221967 129.128033) (width 0.2) (layer "F.Cu") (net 1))
 (segment (start 149.885001 131.1) (end 150.63 131.1) (width 0.3) (layer "F.Cu") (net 1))
 (segment (start 150.71 128.04) (end 151.1175 128.04) (width 0.2) (layer "F.Cu") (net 1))
 (segment (start 150.3 128.45) (end 150.71 128.04) (width 0.2) (layer "F.Cu") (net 1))
 (segment (start 149.885001 130.25) (end 150.6 130.25) (width 0.3) (layer "F.Cu") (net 1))
 (via (at 159.5 123.5) (size 0.65) (drill 0.25) (layers "F.Cu" "B.Cu") (free yes) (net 1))
 (via (at 149.885001 130.25) (size 0.65) (drill 0.25) (layers "F.Cu" "B.Cu") (free yes) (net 1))
 (via (at 150.15 128.45) (size 0.65) (drill 0.25) (layers "F.Cu" "B.Cu") (free yes) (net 1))
 (via (at 149.885001 131.1) (size 0.65) (drill 0.25) (layers "F.Cu" "B.Cu") (free yes) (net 1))
 (via (at 150.05 126.1) (size 0.65) (drill 0.25) (layers "F.Cu" "B.Cu") (free yes) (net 1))
 (via (at 150.15 129.128033) (size 0.65) (drill 0.25) (layers "F.Cu" "B.Cu") (free yes) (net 1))
 (segment (start 161.75 118.74) (end 159.25 116.24) (width 0.15) (layer "F.Cu") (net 19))
 (segment (start 156.17 134.04) (end 161.75 128.46) (width 0.15) (layer "F.Cu") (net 19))
 (segment (start 161.75 128.46) (end 161.75 118.74) (width 0.15) (layer "F.Cu") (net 19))
 (segment (start 157.4 131.5) (end 161 127.9) (width 0.15) (layer "F.Cu") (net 20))
 (segment (start 161 120.53) (end 159.25 118.78) (width 0.15) (layer "F.Cu") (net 20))
 (segment (start 161 127.9) (end 161 120.53) (width 0.15) (layer "F.Cu") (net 20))
 (segment (start 156.17 131.5) (end 157.4 131.5) (width 0.15) (layer "F.Cu") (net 20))
 (segment (start 154.03 128.04) (end 154.55 128.04) (width 0.2) (layer "F.Cu") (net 22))
 (segment (start 154.55 128.04) (end 156.17 126.42) (width 0.2) (layer "F.Cu") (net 22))
 (segment (start 153.21 127.54) (end 153.56 127.19) (width 0.2) (layer "F.Cu") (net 21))
 (segment (start 154.75 125.5) (end 155.25 125) (width 0.2) (layer "F.Cu") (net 21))
 (segment (start 155.25 125) (end 157 125) (width 0.2) (layer "F.Cu") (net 21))
 (segment (start 157.5 125.5) (end 157.5 127.63) (width 0.2) (layer "F.Cu") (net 21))
 (segment (start 154.75 127) (end 154.75 125.5) (width 0.2) (layer "F.Cu") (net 21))
 (segment (start 154.04 127.19) (end 154.56 127.19) (width 0.2) (layer "F.Cu") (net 21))
 (segment (start 154.56 127.19) (end 154.75 127) (width 0.2) (layer "F.Cu") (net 21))
 (segment (start 153.56 127.19) (end 154.04 127.19) (width 0.2) (layer "F.Cu") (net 21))
 (segment (start 152.9425 127.54) (end 153.21 127.54) (width 0.2) (layer "F.Cu") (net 21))
 (segment (start 157 125) (end 157.5 125.5) (width 0.2) (layer "F.Cu") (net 21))
 (segment (start 157.5 127.63) (end 156.17 128.96) (width 0.2) (layer "F.Cu") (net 21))
 (segment (start 140.93 128.96) (end 137.84 128.96) (width 0.2) (layer "F.Cu") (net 10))
 (segment (start 135.3 111.18) (end 135.3 141.66) (width 1.75) (layer "F.Cu") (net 28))
 (segment (start 153.23 105.7) (end 138.1 105.7) (width 1.75) (layer "F.Cu") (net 28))
 (segment (start 156.17 108.64) (end 153.23 105.7) (width 1.75) (layer "F.Cu") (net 28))
 (segment (start 135.3 108.5) (end 135.3 111.18) (width 1.75) (layer "F.Cu") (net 28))
 (segment (start 138.1 105.7) (end 135.3 108.5) (width 1.75) (layer "F.Cu") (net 28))
 (segment (start 140.93 136.58) (end 137.84 136.58) (width 0.2) (layer "F.Cu") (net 13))
 (segment (start 140.93 118.8) (end 137.84 118.8) (width 0.2) (layer "F.Cu") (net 5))
 (segment (start 140.93 139.12) (end 137.84 139.12) (width 0.2) (layer "F.Cu") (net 14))
 (segment (start 140.93 123.88) (end 137.84 123.88) (width 0.2) (layer "F.Cu") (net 8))
 (segment (start 140.93 111.18) (end 137.84 111.18) (width 0.2) (layer "F.Cu") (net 2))
 (segment (start 140.93 121.34) (end 137.84 121.34) (width 0.2) (layer "F.Cu") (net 7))
 (segment (start 140.93 116.26) (end 137.84 116.26) (width 0.2) (layer "F.Cu") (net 4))
 (segment (start 140.93 134.04) (end 137.84 134.04) (width 0.2) (layer "F.Cu") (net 12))
 (segment (start 157.3 124.35) (end 158.15 125.2) (width 0.2) (layer "F.Cu") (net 25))
 (segment (start 156.17 118.8) (end 156.17 118.845) (width 0.2) (layer "F.Cu") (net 25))
 (segment (start 157.3 119.975) (end 157.3 124.35) (width 0.2) (layer "F.Cu") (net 25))
 (segment (start 156.75 130.2) (end 155.55 130.2) (width 0.2) (layer "F.Cu") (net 25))
 (segment (start 158.15 128.8) (end 156.75 130.2) (width 0.2) (layer "F.Cu") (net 25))
 (segment (start 152.15 130.2) (end 152.15 130.035) (width 0.2) (layer "F.Cu") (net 25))
 (segment (start 155.55 130.2) (end 153.851992 131.898008) (width 0.2) (layer "F.Cu") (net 25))
 (segment (start 152.15 130.035) (end 151.78 129.665) (width 0.2) (layer "F.Cu") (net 25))
 (segment (start 156.17 118.845) (end 157.3 119.975) (width 0.2) (layer "F.Cu") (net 25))
 (segment (start 152.751992 130.801992) (end 152.15 130.2) (width 0.2) (layer "F.Cu") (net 25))
 (segment (start 158.15 125.2) (end 158.15 128.8) (width 0.2) (layer "F.Cu") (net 25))
 (segment (start 153.851992 131.898008) (end 153.848008 131.898008) (width 0.2) (layer "F.Cu") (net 25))
 (segment (start 151.78 129.665) (end 151.78 129.2025) (width 0.2) (layer "F.Cu") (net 25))
 (via (at 152.751992 130.801992) (size 0.65) (drill 0.25) (layers "F.Cu" "B.Cu") (free yes) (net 25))
 (via (at 153.848008 131.898008) (size 0.65) (drill 0.25) (layers "F.Cu" "B.Cu") (free yes) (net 25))
 (segment (start 153.848008 131.898008) (end 152.751992 130.801992) (width 0.2) (layer "B.Cu") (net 25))
 (segment (start 140.93 141.66) (end 137.84 141.66) (width 0.2) (layer "F.Cu") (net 15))
 (segment (start 140.93 131.5) (end 137.84 131.5) (width 0.2) (layer "F.Cu") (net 11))
 (segment (start 140.93 113.72) (end 137.84 113.72) (width 0.2) (layer "F.Cu") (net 3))
 (segment (start 140.93 126.42) (end 137.84 126.42) (width 0.2) (layer "F.Cu") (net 9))
 (segment (start 151.28 119.645) (end 154.665 116.26) (width 0.2) (layer "F.Cu") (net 26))
 (segment (start 151.28 126.8775) (end 151.28 119.645) (width 0.2) (layer "F.Cu") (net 26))
 (segment (start 154.665 116.26) (end 156.17 116.26) (width 0.2) (layer "F.Cu") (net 26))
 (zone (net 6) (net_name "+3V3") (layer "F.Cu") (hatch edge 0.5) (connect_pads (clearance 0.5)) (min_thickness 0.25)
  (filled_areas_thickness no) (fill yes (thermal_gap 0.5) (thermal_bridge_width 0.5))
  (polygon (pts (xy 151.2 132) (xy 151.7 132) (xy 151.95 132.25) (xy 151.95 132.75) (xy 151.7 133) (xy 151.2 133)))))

